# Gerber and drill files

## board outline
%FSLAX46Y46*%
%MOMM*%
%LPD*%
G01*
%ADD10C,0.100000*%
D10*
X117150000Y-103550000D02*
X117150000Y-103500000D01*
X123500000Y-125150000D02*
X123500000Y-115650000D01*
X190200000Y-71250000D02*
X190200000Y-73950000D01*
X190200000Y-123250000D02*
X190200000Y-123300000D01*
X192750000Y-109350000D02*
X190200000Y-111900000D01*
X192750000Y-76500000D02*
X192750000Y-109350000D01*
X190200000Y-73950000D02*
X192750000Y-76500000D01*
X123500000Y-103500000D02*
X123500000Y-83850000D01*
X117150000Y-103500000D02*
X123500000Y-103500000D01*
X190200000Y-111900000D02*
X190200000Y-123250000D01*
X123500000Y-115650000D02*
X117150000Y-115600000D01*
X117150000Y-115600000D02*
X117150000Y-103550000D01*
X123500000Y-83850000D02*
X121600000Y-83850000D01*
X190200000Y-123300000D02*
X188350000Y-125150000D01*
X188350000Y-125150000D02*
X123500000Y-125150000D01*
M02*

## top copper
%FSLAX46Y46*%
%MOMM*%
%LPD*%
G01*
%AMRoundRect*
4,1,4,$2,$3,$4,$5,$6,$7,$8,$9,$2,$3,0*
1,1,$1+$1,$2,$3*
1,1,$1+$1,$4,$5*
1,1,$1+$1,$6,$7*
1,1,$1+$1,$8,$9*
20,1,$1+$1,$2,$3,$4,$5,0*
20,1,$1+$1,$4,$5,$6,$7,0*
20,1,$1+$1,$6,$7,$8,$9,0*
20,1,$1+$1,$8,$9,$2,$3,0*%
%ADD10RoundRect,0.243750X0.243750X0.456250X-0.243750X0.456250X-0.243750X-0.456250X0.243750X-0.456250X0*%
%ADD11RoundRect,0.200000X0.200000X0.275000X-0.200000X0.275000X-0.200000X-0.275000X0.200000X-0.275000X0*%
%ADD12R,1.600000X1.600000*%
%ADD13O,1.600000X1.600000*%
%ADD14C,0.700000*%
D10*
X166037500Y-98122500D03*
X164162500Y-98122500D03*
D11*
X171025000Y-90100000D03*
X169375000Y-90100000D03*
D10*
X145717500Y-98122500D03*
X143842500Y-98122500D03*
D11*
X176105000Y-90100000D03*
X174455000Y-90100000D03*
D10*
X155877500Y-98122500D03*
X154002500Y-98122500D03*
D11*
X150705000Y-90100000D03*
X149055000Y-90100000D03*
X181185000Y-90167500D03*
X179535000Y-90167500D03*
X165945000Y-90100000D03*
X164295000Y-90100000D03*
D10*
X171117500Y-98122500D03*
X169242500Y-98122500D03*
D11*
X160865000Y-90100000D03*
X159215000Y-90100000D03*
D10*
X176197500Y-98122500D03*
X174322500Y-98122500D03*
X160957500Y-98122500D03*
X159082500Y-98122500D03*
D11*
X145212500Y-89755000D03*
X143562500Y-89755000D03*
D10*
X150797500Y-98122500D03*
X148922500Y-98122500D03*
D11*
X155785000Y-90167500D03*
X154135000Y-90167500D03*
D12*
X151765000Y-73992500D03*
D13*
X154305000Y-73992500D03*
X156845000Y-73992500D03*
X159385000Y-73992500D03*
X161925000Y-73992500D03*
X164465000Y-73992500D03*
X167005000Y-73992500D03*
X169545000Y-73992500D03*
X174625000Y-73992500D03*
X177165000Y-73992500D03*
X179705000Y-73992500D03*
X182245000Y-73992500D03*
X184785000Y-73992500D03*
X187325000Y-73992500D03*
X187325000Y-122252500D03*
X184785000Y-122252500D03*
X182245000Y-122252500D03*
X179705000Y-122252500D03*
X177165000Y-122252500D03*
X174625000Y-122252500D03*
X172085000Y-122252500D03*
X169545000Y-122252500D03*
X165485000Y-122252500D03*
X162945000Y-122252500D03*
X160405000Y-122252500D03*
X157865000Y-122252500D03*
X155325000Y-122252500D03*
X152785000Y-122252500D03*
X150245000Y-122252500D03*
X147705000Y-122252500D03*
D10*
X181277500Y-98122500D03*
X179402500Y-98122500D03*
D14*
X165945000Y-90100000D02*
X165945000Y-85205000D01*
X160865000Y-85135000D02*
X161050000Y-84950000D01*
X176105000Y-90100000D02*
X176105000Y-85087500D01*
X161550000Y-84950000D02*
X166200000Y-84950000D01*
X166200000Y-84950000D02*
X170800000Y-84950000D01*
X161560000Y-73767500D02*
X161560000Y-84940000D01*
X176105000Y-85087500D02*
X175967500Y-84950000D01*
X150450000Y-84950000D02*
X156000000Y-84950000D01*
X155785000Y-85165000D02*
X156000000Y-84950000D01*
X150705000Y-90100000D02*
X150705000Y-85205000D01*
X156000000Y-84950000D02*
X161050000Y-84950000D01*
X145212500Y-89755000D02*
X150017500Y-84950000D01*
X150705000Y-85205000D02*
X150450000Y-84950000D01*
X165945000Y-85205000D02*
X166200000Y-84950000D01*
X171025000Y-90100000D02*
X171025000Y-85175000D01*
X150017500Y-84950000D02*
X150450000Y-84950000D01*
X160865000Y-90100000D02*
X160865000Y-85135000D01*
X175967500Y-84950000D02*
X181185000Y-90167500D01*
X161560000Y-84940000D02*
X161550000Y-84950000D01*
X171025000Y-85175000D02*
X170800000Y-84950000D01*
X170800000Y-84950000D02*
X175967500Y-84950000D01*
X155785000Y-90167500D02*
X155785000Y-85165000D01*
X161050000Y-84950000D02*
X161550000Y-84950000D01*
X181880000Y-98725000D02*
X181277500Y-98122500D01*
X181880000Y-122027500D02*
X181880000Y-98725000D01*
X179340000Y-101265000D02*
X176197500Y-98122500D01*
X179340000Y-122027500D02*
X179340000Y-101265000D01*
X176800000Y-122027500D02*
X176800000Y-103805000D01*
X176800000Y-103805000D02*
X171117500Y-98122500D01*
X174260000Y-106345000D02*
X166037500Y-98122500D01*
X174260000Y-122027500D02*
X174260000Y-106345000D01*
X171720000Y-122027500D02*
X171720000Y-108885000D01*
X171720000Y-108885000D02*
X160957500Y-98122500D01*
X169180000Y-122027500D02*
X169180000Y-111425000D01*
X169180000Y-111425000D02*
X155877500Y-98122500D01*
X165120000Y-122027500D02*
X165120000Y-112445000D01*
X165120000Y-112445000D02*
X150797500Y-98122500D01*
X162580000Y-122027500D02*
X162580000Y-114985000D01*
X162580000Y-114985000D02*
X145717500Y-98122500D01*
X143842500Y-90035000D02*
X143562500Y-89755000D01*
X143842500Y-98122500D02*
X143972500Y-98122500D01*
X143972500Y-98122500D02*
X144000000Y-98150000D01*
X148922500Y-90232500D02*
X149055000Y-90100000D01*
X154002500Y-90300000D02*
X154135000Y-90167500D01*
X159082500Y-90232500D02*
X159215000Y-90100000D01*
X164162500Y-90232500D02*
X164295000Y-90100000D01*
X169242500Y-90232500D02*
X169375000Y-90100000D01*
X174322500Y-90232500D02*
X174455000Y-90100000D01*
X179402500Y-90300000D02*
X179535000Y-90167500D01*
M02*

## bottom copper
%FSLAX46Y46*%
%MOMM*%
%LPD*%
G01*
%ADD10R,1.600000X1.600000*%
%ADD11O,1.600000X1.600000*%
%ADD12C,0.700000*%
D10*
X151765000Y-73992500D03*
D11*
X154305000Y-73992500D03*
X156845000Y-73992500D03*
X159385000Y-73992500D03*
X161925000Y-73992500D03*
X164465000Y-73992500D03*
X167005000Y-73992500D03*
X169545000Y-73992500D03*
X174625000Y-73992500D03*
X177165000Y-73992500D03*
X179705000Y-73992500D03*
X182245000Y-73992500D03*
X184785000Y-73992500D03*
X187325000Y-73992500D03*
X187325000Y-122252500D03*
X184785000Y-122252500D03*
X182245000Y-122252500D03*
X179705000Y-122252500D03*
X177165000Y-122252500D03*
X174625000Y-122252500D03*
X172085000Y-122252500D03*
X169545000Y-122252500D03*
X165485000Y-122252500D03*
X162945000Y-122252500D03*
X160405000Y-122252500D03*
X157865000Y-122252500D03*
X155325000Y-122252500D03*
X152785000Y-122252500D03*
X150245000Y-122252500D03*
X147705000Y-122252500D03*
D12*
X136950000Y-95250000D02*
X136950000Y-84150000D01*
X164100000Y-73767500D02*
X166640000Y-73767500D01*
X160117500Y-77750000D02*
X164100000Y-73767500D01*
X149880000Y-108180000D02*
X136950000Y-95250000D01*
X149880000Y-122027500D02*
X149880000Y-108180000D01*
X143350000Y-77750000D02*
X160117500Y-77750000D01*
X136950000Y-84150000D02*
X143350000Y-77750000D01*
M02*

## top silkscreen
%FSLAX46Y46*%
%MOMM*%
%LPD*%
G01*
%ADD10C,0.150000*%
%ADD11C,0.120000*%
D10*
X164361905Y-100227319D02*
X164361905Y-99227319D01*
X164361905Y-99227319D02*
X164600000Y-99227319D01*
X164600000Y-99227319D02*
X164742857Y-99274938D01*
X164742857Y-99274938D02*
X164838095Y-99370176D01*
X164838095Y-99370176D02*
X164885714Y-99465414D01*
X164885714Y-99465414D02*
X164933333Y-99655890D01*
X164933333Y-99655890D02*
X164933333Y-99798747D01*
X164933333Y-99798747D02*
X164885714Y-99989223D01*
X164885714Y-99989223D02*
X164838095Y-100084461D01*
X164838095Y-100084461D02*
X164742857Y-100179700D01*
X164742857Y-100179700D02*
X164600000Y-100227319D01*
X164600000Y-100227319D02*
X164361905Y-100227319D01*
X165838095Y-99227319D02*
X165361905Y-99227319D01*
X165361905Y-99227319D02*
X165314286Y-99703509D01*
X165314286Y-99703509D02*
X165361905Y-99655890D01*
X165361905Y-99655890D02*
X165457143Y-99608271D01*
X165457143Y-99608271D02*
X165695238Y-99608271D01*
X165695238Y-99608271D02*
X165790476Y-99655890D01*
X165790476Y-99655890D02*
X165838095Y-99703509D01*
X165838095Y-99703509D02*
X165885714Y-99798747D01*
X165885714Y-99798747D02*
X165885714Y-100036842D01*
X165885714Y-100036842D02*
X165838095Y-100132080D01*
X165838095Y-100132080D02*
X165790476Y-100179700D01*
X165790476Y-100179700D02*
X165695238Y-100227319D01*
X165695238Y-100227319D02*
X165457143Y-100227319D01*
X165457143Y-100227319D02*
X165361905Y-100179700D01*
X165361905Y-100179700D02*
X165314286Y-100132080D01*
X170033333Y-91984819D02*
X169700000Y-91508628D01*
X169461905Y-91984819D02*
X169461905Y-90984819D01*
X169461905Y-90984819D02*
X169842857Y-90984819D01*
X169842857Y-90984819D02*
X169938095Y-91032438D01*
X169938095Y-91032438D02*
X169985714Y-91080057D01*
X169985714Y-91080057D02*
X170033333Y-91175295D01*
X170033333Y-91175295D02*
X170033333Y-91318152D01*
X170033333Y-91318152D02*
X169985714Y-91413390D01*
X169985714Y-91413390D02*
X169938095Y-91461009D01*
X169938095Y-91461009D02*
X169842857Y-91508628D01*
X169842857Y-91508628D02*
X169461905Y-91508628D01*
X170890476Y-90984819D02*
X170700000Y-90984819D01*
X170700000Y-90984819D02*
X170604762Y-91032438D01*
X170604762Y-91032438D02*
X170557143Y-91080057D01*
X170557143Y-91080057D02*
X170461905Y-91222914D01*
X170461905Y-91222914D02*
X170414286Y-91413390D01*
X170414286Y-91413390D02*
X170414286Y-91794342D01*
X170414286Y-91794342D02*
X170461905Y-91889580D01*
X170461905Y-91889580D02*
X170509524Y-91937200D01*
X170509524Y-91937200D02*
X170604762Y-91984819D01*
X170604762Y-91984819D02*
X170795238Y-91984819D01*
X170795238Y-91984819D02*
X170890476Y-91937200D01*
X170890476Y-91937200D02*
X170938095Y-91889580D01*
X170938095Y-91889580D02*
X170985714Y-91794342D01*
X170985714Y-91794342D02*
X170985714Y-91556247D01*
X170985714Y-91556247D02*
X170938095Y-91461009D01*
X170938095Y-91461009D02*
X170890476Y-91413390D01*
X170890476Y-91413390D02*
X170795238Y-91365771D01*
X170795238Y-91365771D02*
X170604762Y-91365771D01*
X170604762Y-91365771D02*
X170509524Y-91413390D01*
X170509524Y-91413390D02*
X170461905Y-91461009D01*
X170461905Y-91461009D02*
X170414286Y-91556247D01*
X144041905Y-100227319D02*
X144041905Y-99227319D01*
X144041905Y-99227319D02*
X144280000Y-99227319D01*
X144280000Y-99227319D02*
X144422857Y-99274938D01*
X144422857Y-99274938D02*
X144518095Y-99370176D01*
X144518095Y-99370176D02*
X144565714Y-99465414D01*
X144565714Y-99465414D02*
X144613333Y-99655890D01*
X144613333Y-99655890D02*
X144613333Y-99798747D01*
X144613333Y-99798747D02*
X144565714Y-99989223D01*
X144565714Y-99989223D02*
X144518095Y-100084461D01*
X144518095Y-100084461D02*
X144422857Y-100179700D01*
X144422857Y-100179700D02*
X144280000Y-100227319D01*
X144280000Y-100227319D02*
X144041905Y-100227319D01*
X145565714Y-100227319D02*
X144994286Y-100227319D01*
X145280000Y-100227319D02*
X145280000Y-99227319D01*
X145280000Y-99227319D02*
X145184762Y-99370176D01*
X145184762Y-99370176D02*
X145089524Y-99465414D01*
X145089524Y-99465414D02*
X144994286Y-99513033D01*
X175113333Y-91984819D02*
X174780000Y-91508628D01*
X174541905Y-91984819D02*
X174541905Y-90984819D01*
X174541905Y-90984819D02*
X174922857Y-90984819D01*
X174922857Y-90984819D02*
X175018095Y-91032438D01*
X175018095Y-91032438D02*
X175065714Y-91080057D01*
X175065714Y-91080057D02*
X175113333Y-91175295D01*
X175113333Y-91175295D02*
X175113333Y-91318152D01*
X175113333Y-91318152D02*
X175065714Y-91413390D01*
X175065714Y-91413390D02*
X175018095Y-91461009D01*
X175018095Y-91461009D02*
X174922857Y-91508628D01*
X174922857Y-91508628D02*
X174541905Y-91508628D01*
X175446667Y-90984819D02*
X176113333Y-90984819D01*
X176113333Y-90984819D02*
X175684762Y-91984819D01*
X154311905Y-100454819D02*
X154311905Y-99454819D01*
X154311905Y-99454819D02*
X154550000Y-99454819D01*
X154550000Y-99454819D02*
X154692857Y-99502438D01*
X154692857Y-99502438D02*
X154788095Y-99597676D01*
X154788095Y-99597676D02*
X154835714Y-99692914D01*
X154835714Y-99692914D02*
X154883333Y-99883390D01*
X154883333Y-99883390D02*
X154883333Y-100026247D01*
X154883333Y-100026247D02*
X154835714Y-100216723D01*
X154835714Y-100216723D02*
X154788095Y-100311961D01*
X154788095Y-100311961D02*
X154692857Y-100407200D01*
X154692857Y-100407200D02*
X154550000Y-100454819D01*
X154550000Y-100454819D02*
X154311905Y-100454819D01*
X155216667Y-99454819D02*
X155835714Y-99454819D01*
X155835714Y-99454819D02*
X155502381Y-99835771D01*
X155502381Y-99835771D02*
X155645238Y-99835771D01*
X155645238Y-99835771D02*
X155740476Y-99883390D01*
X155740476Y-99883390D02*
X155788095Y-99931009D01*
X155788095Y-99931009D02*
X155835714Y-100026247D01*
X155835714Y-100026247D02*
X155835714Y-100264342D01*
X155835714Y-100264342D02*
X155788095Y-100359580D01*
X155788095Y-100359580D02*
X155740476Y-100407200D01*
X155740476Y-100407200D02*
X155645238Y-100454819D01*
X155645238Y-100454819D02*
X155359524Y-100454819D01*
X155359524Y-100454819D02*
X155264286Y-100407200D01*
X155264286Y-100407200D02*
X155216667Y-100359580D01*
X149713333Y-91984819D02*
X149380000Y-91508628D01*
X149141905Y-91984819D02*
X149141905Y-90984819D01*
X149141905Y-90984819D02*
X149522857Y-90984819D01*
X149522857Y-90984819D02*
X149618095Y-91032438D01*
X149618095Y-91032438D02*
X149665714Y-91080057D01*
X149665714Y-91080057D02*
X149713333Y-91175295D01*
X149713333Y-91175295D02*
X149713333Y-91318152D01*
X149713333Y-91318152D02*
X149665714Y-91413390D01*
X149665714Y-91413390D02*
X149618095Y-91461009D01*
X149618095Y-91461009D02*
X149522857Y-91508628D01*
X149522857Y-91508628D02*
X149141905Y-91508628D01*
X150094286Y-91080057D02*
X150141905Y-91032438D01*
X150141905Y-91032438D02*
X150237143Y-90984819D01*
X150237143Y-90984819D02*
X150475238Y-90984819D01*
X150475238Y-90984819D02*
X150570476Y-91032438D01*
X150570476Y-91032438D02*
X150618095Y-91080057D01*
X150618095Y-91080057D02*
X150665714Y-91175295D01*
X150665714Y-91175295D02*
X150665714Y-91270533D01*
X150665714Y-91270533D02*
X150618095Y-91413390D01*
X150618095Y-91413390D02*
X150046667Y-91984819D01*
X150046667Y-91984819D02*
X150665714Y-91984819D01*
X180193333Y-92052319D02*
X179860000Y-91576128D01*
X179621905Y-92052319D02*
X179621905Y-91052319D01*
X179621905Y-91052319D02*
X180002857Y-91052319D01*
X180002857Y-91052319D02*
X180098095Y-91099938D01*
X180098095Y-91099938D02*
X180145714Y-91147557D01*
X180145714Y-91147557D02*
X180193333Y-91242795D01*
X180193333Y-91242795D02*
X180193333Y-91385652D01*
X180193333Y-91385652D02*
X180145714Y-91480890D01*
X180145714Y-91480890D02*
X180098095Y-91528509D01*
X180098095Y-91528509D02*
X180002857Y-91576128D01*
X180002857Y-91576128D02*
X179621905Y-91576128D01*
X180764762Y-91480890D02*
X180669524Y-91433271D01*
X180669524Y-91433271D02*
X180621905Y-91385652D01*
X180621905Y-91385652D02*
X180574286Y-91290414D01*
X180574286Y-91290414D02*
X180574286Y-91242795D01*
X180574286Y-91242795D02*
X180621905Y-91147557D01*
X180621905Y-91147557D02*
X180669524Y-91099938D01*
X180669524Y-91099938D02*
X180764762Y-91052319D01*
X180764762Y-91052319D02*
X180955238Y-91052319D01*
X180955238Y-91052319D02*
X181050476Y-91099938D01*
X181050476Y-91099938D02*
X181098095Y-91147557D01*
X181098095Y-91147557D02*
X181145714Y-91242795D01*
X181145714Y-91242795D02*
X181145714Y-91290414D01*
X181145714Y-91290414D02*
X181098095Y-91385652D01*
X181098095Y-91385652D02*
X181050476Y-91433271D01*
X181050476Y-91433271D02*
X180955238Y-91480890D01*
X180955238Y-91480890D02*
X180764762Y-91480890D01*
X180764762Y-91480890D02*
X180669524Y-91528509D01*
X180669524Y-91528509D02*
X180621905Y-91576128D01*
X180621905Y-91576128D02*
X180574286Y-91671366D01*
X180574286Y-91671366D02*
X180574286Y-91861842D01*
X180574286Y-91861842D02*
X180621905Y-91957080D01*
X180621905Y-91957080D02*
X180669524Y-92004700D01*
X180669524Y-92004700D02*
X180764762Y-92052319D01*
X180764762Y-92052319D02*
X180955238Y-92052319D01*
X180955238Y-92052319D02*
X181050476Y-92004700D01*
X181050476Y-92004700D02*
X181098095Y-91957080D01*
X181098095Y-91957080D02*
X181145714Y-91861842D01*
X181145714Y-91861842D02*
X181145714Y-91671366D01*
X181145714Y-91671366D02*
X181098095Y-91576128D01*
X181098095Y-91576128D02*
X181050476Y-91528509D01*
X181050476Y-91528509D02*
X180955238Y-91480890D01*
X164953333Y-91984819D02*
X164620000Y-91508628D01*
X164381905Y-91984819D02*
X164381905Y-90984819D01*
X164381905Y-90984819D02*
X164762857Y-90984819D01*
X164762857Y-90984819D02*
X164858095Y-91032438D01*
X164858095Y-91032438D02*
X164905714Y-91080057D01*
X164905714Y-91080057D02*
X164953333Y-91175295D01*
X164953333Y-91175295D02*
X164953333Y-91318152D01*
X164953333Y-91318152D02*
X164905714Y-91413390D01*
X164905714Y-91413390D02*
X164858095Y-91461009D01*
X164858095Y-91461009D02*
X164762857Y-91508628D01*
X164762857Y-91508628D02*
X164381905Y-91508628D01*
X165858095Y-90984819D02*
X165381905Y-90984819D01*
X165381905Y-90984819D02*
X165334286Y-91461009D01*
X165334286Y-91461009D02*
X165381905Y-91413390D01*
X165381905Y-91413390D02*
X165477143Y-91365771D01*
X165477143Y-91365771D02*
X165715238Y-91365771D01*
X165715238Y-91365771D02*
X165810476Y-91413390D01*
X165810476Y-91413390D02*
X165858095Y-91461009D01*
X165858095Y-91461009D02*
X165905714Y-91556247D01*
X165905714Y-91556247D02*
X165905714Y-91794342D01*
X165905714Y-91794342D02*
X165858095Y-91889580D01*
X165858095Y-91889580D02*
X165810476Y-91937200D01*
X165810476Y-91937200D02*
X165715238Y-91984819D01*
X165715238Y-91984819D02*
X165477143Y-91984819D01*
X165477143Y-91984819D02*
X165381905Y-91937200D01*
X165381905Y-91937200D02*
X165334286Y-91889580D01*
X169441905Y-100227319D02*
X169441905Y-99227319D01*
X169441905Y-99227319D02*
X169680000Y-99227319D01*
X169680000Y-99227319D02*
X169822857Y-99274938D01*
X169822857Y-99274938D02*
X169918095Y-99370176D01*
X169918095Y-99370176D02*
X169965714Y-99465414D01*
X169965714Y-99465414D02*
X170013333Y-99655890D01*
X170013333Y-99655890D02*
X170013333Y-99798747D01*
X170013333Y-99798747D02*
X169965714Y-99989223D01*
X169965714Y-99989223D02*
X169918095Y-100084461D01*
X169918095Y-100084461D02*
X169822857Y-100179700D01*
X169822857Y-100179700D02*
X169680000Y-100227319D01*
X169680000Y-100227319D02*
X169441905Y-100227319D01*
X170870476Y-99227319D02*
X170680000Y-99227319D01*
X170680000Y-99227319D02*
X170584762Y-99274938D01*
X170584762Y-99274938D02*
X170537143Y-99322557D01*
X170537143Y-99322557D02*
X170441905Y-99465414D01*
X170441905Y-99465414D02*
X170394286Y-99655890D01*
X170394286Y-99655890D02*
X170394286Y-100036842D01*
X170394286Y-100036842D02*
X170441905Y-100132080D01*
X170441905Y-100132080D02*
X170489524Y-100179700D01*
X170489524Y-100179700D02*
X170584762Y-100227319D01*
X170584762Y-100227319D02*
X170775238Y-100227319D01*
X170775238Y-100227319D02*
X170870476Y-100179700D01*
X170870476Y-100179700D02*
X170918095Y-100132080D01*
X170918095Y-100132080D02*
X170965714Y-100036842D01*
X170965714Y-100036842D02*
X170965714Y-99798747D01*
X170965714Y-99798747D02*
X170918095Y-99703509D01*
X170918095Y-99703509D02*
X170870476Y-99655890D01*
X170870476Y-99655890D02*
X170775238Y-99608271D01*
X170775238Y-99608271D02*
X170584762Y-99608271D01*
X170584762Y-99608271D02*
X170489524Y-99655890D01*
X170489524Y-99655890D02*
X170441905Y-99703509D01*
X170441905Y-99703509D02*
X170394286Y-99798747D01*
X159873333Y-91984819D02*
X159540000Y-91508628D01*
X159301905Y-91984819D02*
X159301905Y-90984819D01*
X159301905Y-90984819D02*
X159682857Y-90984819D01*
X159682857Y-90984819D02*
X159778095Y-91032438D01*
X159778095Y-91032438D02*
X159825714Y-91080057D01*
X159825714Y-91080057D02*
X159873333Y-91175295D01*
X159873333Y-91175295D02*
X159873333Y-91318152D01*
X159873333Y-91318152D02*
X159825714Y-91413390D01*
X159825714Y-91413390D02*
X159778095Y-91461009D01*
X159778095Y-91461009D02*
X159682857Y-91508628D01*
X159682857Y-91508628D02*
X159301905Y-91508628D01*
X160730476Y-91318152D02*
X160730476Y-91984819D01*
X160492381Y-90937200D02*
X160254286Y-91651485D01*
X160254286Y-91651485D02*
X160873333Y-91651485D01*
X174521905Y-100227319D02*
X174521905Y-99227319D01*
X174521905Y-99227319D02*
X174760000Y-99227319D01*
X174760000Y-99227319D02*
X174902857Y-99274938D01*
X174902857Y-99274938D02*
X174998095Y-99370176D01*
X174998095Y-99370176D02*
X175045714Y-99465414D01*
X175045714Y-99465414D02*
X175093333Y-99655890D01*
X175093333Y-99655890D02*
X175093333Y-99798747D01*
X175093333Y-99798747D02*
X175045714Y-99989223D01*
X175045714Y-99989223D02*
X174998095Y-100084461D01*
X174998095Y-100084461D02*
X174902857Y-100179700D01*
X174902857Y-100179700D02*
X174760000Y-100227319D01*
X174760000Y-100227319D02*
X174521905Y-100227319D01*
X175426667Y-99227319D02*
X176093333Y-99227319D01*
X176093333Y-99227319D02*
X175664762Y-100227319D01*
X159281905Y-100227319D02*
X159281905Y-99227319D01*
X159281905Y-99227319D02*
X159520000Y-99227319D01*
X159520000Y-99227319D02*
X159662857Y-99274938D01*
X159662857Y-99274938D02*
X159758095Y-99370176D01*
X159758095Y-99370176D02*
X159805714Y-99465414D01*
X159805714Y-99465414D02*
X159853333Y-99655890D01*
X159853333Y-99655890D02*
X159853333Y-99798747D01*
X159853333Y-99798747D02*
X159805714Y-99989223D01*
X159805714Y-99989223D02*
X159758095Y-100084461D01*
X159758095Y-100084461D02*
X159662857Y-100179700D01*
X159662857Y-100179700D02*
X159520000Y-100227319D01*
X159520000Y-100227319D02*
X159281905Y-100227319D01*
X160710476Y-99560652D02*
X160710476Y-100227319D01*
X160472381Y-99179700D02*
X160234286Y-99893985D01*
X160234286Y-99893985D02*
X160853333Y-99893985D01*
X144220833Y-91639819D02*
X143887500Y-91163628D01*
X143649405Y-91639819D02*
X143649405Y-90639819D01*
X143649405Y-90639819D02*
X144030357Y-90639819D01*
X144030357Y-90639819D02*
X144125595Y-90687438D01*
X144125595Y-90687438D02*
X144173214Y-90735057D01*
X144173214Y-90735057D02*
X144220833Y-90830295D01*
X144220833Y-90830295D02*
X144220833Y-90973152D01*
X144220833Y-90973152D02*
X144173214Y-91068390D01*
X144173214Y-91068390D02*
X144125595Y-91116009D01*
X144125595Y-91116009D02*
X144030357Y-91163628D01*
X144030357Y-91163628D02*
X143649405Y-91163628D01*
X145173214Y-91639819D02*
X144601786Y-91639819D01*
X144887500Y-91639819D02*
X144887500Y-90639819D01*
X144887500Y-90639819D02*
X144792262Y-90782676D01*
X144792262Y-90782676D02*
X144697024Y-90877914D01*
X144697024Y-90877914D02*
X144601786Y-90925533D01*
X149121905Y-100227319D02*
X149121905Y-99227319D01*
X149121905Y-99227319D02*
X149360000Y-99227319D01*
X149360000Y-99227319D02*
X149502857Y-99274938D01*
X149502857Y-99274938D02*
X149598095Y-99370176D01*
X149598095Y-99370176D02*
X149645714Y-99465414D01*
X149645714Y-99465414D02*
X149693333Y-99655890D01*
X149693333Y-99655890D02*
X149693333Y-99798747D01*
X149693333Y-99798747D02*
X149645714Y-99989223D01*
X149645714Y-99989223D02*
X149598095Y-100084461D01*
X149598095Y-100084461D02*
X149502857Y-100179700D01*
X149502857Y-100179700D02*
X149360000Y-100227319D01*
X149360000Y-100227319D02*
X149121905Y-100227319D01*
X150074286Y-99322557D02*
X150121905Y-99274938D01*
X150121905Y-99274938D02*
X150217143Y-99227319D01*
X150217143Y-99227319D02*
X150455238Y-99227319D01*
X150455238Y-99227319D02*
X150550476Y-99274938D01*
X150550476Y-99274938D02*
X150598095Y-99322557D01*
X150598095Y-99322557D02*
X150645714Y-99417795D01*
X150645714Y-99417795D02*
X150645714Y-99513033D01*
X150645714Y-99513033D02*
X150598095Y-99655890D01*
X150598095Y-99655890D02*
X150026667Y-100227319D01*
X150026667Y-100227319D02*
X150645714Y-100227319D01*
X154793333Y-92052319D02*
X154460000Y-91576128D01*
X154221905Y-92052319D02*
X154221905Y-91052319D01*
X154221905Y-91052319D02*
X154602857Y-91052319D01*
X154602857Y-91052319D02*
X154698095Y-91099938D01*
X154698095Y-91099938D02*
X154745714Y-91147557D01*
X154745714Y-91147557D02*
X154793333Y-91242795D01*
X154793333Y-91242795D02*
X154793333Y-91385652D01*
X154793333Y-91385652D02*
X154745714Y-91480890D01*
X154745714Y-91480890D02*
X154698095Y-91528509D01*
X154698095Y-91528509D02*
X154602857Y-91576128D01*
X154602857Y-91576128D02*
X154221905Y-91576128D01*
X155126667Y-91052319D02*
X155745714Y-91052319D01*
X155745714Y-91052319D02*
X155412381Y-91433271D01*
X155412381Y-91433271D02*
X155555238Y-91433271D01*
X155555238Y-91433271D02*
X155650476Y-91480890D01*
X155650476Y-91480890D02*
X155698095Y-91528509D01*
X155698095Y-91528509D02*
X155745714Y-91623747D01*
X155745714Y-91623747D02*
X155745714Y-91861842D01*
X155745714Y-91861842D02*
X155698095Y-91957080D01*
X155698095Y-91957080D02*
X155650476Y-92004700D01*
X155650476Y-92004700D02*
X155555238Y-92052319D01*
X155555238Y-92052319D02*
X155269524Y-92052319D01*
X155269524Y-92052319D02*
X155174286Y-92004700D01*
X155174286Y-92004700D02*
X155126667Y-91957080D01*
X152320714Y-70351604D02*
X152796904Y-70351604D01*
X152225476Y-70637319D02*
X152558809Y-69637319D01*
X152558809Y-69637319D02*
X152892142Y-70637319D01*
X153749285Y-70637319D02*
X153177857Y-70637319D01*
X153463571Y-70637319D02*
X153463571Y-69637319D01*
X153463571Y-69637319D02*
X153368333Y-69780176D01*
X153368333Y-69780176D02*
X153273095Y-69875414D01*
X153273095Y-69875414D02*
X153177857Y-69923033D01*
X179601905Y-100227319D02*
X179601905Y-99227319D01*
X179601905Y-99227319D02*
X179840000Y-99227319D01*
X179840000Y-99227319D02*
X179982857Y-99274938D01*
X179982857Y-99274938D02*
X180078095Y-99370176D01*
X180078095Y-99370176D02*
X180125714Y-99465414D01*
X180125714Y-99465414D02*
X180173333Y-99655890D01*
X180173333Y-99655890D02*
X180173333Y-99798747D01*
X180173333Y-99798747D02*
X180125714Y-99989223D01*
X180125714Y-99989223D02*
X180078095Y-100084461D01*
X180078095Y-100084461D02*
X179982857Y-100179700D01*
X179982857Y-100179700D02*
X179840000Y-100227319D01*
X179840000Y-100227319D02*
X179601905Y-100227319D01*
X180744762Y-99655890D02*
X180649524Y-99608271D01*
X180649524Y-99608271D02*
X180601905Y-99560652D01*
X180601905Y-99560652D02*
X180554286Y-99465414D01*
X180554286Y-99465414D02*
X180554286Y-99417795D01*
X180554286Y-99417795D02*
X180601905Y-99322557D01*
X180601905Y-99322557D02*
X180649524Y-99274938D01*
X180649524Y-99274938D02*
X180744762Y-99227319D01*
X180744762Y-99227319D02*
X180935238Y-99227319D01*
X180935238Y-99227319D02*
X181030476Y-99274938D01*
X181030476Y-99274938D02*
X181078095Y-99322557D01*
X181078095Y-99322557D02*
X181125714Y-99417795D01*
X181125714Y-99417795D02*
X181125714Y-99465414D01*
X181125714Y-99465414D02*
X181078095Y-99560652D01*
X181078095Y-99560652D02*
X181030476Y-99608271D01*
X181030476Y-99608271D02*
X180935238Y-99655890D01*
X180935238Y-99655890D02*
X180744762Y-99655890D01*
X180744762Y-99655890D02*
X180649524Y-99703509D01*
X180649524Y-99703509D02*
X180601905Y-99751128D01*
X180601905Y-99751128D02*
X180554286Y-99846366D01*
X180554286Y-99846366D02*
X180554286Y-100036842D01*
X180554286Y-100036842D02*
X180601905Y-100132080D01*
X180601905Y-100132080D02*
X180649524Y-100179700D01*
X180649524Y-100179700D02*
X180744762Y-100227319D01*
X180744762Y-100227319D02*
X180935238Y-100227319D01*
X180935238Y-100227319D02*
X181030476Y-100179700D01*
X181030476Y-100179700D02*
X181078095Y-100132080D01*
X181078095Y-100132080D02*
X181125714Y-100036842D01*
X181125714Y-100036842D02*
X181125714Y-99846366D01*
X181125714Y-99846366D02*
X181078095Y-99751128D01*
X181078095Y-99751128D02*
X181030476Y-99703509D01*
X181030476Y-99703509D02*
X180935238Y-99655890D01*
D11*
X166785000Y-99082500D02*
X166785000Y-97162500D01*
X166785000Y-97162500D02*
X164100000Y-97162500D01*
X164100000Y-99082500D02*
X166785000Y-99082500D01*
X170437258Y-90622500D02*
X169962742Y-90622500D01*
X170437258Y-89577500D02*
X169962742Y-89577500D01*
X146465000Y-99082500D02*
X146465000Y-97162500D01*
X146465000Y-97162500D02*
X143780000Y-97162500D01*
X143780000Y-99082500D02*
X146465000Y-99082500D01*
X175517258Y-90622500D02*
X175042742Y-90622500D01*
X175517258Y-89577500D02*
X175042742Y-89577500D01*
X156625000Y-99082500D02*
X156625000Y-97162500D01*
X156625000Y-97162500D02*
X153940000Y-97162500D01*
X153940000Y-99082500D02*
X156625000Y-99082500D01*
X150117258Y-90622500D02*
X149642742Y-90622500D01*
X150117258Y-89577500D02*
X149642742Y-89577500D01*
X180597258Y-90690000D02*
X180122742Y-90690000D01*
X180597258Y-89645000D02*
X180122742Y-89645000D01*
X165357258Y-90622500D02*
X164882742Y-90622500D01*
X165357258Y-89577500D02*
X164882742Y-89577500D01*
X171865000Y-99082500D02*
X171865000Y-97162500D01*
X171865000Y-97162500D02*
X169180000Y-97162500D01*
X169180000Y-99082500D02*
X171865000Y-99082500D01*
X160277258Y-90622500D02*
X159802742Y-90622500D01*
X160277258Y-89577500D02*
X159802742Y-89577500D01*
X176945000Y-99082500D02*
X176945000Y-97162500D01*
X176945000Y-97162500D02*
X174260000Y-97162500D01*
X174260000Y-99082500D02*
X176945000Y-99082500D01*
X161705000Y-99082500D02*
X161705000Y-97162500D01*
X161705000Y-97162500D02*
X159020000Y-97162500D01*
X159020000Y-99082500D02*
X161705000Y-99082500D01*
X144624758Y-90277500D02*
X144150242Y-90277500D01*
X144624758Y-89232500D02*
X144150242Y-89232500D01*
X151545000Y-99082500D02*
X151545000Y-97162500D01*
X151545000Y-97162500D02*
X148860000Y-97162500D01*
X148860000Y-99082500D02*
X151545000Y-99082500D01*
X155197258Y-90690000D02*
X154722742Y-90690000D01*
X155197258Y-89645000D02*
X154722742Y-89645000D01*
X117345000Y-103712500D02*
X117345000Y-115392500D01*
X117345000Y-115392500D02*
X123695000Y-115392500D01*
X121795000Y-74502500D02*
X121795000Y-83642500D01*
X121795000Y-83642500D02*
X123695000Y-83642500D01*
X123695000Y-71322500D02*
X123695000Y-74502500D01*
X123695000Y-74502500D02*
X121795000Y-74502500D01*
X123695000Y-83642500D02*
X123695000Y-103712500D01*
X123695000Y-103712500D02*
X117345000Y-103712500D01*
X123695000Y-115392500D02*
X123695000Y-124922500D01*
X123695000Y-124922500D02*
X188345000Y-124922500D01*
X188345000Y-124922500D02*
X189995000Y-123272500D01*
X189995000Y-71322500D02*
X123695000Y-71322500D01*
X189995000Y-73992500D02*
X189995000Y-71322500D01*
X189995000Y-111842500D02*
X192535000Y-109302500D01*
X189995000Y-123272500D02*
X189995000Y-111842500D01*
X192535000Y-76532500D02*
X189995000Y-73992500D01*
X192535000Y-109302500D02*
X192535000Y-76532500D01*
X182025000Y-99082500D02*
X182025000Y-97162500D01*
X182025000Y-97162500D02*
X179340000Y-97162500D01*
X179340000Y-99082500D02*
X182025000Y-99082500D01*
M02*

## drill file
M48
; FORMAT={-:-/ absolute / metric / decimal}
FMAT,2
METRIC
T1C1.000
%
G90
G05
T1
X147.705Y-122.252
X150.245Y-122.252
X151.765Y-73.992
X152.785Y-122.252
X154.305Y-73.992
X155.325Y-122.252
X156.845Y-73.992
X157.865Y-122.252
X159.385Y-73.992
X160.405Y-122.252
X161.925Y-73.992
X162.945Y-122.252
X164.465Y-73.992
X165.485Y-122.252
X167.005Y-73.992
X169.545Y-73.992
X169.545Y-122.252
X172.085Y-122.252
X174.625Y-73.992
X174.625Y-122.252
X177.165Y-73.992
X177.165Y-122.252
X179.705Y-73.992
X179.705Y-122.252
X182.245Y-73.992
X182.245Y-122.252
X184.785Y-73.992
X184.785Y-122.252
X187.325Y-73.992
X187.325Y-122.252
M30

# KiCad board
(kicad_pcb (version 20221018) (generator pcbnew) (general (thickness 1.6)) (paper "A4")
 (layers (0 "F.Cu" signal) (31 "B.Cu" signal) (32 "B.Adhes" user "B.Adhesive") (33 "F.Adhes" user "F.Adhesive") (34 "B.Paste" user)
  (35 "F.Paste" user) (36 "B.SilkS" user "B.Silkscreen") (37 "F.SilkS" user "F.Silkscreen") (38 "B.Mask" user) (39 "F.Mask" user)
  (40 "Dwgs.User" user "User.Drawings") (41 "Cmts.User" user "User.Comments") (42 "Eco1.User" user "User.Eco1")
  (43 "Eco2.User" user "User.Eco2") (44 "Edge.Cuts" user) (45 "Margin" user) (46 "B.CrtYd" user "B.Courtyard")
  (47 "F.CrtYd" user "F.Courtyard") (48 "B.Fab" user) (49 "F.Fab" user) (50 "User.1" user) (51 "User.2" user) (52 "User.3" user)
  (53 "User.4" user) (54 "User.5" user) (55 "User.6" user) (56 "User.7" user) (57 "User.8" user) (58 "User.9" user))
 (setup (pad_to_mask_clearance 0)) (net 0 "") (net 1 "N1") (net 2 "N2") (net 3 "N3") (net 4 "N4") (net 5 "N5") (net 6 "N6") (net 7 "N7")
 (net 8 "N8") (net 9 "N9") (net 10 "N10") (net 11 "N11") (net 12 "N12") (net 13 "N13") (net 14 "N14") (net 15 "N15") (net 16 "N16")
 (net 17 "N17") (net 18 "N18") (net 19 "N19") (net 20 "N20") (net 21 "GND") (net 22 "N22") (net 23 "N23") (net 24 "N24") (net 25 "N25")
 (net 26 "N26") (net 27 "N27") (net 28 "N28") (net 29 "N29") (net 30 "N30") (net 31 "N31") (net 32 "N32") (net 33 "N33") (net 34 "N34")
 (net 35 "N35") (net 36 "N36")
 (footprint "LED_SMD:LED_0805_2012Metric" (layer "F.Cu") (at 165.1 98.1225 180)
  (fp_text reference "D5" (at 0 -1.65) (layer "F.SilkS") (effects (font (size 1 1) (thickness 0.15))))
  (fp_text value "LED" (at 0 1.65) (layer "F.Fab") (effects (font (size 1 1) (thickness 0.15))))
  (fp_line (start -1.685 -0.96) (end -1.685 0.96) (stroke (width 0.12) (type solid)) (layer "F.SilkS"))
  (fp_line (start -1.685 0.96) (end 1 0.96) (stroke (width 0.12) (type solid)) (layer "F.SilkS"))
  (fp_line (start 1 -0.96) (end -1.685 -0.96) (stroke (width 0.12) (type solid)) (layer "F.SilkS"))
  (pad "1" smd roundrect (at -0.9375 0 180) (size 0.975 1.4) (layers "F.Cu" "F.Paste" "F.Mask") (roundrect_rratio 0.25) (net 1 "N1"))
  (pad "2" smd roundrect (at 0.9375 0 180) (size 0.975 1.4) (layers "F.Cu" "F.Paste" "F.Mask") (roundrect_rratio 0.25) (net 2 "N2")))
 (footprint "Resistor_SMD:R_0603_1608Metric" (layer "F.Cu") (at 170.2 90.1 180)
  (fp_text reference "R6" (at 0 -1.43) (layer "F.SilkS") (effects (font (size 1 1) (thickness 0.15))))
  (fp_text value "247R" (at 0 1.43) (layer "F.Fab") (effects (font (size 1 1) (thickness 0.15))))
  (fp_line (start -0.237258 -0.5225) (end 0.237258 -0.5225) (stroke (width 0.12) (type solid)) (layer "F.SilkS"))
  (fp_line (start -0.237258 0.5225) (end 0.237258 0.5225) (stroke (width 0.12) (type solid)) (layer "F.SilkS"))
  (pad "1" smd roundrect (at -0.825 0 180) (size 0.8 0.95) (layers "F.Cu" "F.Paste" "F.Mask") (roundrect_rratio 0.25) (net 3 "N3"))
  (pad "2" smd roundrect (at 0.825 0 180) (size 0.8 0.95) (layers "F.Cu" "F.Paste" "F.Mask") (roundrect_rratio 0.25) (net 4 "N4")))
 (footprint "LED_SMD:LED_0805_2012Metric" (layer "F.Cu") (at 144.78 98.1225 180)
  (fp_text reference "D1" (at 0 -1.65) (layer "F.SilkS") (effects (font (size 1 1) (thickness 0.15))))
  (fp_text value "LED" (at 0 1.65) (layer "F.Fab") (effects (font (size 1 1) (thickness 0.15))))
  (fp_line (start -1.685 -0.96) (end -1.685 0.96) (stroke (width 0.12) (type solid)) (layer "F.SilkS"))
  (fp_line (start -1.685 0.96) (end 1 0.96) (stroke (width 0.12) (type solid)) (layer "F.SilkS"))
  (fp_line (start 1 -0.96) (end -1.685 -0.96) (stroke (width 0.12) (type solid)) (layer "F.SilkS"))
  (pad "1" smd roundrect (at -0.9375 0 180) (size 0.975 1.4) (layers "F.Cu" "F.Paste" "F.Mask") (roundrect_rratio 0.25) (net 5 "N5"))
  (pad "2" smd roundrect (at 0.9375 0 180) (size 0.975 1.4) (layers "F.Cu" "F.Paste" "F.Mask") (roundrect_rratio 0.25) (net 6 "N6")))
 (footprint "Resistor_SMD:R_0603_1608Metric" (layer "F.Cu") (at 175.28 90.1 180)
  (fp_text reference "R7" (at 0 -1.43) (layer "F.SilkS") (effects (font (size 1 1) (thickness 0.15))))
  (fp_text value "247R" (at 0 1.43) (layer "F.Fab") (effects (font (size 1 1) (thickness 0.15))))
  (fp_line (start -0.237258 -0.5225) (end 0.237258 -0.5225) (stroke (width 0.12) (type solid)) (layer "F.SilkS"))
  (fp_line (start -0.237258 0.5225) (end 0.237258 0.5225) (stroke (width 0.12) (type solid)) (layer "F.SilkS"))
  (pad "1" smd roundrect (at -0.825 0 180) (size 0.8 0.95) (layers "F.Cu" "F.Paste" "F.Mask") (roundrect_rratio 0.25) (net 3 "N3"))
  (pad "2" smd roundrect (at 0.825 0 180) (size 0.8 0.95) (layers "F.Cu" "F.Paste" "F.Mask") (roundrect_rratio 0.25) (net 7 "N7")))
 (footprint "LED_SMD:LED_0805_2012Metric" (layer "F.Cu") (at 154.94 98.1225 180)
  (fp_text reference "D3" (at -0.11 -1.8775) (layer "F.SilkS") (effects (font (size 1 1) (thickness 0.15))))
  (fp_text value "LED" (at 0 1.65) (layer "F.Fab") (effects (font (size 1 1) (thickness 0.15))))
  (fp_line (start -1.685 -0.96) (end -1.685 0.96) (stroke (width 0.12) (type solid)) (layer "F.SilkS"))
  (fp_line (start -1.685 0.96) (end 1 0.96) (stroke (width 0.12) (type solid)) (layer "F.SilkS"))
  (fp_line (start 1 -0.96) (end -1.685 -0.96) (stroke (width 0.12) (type solid)) (layer "F.SilkS"))
  (pad "1" smd roundrect (at -0.9375 0 180) (size 0.975 1.4) (layers "F.Cu" "F.Paste" "F.Mask") (roundrect_rratio 0.25) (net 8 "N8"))
  (pad "2" smd roundrect (at 0.9375 0 180) (size 0.975 1.4) (layers "F.Cu" "F.Paste" "F.Mask") (roundrect_rratio 0.25) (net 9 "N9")))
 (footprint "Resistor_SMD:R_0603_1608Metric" (layer "F.Cu") (at 149.88 90.1 180)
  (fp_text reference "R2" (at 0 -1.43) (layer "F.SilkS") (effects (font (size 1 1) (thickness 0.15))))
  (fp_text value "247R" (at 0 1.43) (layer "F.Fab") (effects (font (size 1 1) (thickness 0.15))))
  (fp_line (start -0.237258 -0.5225) (end 0.237258 -0.5225) (stroke (width 0.12) (type solid)) (layer "F.SilkS"))
  (fp_line (start -0.237258 0.5225) (end 0.237258 0.5225) (stroke (width 0.12) (type solid)) (layer "F.SilkS"))
  (pad "1" smd roundrect (at -0.825 0 180) (size 0.8 0.95) (layers "F.Cu" "F.Paste" "F.Mask") (roundrect_rratio 0.25) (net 3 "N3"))
  (pad "2" smd roundrect (at 0.825 0 180) (size 0.8 0.95) (layers "F.Cu" "F.Paste" "F.Mask") (roundrect_rratio 0.25) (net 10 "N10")))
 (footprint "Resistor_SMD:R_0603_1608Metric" (layer "F.Cu") (at 180.36 90.1675 180)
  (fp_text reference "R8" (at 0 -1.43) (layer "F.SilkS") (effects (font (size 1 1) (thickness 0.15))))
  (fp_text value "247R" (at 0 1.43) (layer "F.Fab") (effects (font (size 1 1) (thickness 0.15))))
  (fp_line (start -0.237258 -0.5225) (end 0.237258 -0.5225) (stroke (width 0.12) (type solid)) (layer "F.SilkS"))
  (fp_line (start -0.237258 0.5225) (end 0.237258 0.5225) (stroke (width 0.12) (type solid)) (layer "F.SilkS"))
  (pad "1" smd roundrect (at -0.825 0 180) (size 0.8 0.95) (layers "F.Cu" "F.Paste" "F.Mask") (roundrect_rratio 0.25) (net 3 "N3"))
  (pad "2" smd roundrect (at 0.825 0 180) (size 0.8 0.95) (layers "F.Cu" "F.Paste" "F.Mask") (roundrect_rratio 0.25) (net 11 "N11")))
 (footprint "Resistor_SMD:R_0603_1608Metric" (layer "F.Cu") (at 165.12 90.1 180)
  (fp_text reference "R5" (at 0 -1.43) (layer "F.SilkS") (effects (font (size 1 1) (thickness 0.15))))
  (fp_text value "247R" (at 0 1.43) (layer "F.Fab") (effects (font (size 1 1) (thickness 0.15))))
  (fp_line (start -0.237258 -0.5225) (end 0.237258 -0.5225) (stroke (width 0.12) (type solid)) (layer "F.SilkS"))
  (fp_line (start -0.237258 0.5225) (end 0.237258 0.5225) (stroke (width 0.12) (type solid)) (layer "F.SilkS"))
  (pad "1" smd roundrect (at -0.825 0 180) (size 0.8 0.95) (layers "F.Cu" "F.Paste" "F.Mask") (roundrect_rratio 0.25) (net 3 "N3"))
  (pad "2" smd roundrect (at 0.825 0 180) (size 0.8 0.95) (layers "F.Cu" "F.Paste" "F.Mask") (roundrect_rratio 0.25) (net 2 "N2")))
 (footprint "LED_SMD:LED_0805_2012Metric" (layer "F.Cu") (at 170.18 98.1225 180)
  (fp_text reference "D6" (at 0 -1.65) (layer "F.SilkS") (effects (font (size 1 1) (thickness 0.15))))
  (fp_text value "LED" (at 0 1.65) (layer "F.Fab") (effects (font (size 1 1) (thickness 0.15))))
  (fp_line (start -1.685 -0.96) (end -1.685 0.96) (stroke (width 0.12) (type solid)) (layer "F.SilkS"))
  (fp_line (start -1.685 0.96) (end 1 0.96) (stroke (width 0.12) (type solid)) (layer "F.SilkS"))
  (fp_line (start 1 -0.96) (end -1.685 -0.96) (stroke (width 0.12) (type solid)) (layer "F.SilkS"))
  (pad "1" smd roundrect (at -0.9375 0 180) (size 0.975 1.4) (layers "F.Cu" "F.Paste" "F.Mask") (roundrect_rratio 0.25) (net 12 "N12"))
  (pad "2" smd roundrect (at 0.9375 0 180) (size 0.975 1.4) (layers "F.Cu" "F.Paste" "F.Mask") (roundrect_rratio 0.25) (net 4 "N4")))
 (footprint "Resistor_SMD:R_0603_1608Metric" (layer "F.Cu") (at 160.04 90.1 180)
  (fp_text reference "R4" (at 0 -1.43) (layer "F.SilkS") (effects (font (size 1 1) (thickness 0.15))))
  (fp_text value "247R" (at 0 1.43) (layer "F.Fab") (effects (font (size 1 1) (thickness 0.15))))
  (fp_line (start -0.237258 -0.5225) (end 0.237258 -0.5225) (stroke (width 0.12) (type solid)) (layer "F.SilkS"))
  (fp_line (start -0.237258 0.5225) (end 0.237258 0.5225) (stroke (width 0.12) (type solid)) (layer "F.SilkS"))
  (pad "1" smd roundrect (at -0.825 0 180) (size 0.8 0.95) (layers "F.Cu" "F.Paste" "F.Mask") (roundrect_rratio 0.25) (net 3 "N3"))
  (pad "2" smd roundrect (at 0.825 0 180) (size 0.8 0.95) (layers "F.Cu" "F.Paste" "F.Mask") (roundrect_rratio 0.25) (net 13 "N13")))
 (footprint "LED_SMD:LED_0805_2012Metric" (layer "F.Cu") (at 175.26 98.1225 180)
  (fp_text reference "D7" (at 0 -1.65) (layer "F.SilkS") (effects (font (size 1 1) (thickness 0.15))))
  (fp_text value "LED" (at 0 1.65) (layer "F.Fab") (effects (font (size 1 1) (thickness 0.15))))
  (fp_line (start -1.685 -0.96) (end -1.685 0.96) (stroke (width 0.12) (type solid)) (layer "F.SilkS"))
  (fp_line (start -1.685 0.96) (end 1 0.96) (stroke (width 0.12) (type solid)) (layer "F.SilkS"))
  (fp_line (start 1 -0.96) (end -1.685 -0.96) (stroke (width 0.12) (type solid)) (layer "F.SilkS"))
  (pad "1" smd roundrect (at -0.9375 0 180) (size 0.975 1.4) (layers "F.Cu" "F.Paste" "F.Mask") (roundrect_rratio 0.25) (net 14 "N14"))
  (pad "2" smd roundrect (at 0.9375 0 180) (size 0.975 1.4) (layers "F.Cu" "F.Paste" "F.Mask") (roundrect_rratio 0.25) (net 7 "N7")))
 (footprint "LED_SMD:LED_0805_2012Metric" (layer "F.Cu") (at 160.02 98.1225 180)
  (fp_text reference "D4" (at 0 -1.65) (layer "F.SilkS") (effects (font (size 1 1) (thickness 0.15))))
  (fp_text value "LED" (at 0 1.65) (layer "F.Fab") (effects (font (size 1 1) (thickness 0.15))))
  (fp_line (start -1.685 -0.96) (end -1.685 0.96) (stroke (width 0.12) (type solid)) (layer "F.SilkS"))
  (fp_line (start -1.685 0.96) (end 1 0.96) (stroke (width 0.12) (type solid)) (layer "F.SilkS"))
  (fp_line (start 1 -0.96) (end -1.685 -0.96) (stroke (width 0.12) (type solid)) (layer "F.SilkS"))
  (pad "1" smd roundrect (at -0.9375 0 180) (size 0.975 1.4) (layers "F.Cu" "F.Paste" "F.Mask") (roundrect_rratio 0.25) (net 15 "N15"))
  (pad "2" smd roundrect (at 0.9375 0 180) (size 0.975 1.4) (layers "F.Cu" "F.Paste" "F.Mask") (roundrect_rratio 0.25) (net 13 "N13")))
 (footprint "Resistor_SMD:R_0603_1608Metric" (layer "F.Cu") (at 144.3875 89.755 180)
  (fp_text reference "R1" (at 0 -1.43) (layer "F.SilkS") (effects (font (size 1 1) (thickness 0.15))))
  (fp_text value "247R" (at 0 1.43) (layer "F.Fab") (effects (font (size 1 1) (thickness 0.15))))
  (fp_line (start -0.237258 -0.5225) (end 0.237258 -0.5225) (stroke (width 0.12) (type solid)) (layer "F.SilkS"))
  (fp_line (start -0.237258 0.5225) (end 0.237258 0.5225) (stroke (width 0.12) (type solid)) (layer "F.SilkS"))
  (pad "1" smd roundrect (at -0.825 0 180) (size 0.8 0.95) (layers "F.Cu" "F.Paste" "F.Mask") (roundrect_rratio 0.25) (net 3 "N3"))
  (pad "2" smd roundrect (at 0.825 0 180) (size 0.8 0.95) (layers "F.Cu" "F.Paste" "F.Mask") (roundrect_rratio 0.25) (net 6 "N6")))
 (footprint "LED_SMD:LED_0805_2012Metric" (layer "F.Cu") (at 149.86 98.1225 180)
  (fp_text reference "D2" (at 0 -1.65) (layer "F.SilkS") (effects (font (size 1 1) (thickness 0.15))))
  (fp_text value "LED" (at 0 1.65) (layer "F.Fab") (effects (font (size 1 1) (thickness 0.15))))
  (fp_line (start -1.685 -0.96) (end -1.685 0.96) (stroke (width 0.12) (type solid)) (layer "F.SilkS"))
  (fp_line (start -1.685 0.96) (end 1 0.96) (stroke (width 0.12) (type solid)) (layer "F.SilkS"))
  (fp_line (start 1 -0.96) (end -1.685 -0.96) (stroke (width 0.12) (type solid)) (layer "F.SilkS"))
  (pad "1" smd roundrect (at -0.9375 0 180) (size 0.975 1.4) (layers "F.Cu" "F.Paste" "F.Mask") (roundrect_rratio 0.25) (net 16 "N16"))
  (pad "2" smd roundrect (at 0.9375 0 180) (size 0.975 1.4) (layers "F.Cu" "F.Paste" "F.Mask") (roundrect_rratio 0.25) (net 10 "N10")))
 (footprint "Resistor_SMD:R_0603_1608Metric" (layer "F.Cu") (at 154.96 90.1675 180)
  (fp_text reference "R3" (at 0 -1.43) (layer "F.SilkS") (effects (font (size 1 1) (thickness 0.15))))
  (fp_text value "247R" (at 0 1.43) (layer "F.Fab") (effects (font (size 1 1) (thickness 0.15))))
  (fp_line (start -0.237258 -0.5225) (end 0.237258 -0.5225) (stroke (width 0.12) (type solid)) (layer "F.SilkS"))
  (fp_line (start -0.237258 0.5225) (end 0.237258 0.5225) (stroke (width 0.12) (type solid)) (layer "F.SilkS"))
  (pad "1" smd roundrect (at -0.825 0 180) (size 0.8 0.95) (layers "F.Cu" "F.Paste" "F.Mask") (roundrect_rratio 0.25) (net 3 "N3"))
  (pad "2" smd roundrect (at 0.825 0 180) (size 0.8 0.95) (layers "F.Cu" "F.Paste" "F.Mask") (roundrect_rratio 0.25) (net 9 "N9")))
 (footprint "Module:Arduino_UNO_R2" (layer "F.Cu") (at 151.765 73.9925)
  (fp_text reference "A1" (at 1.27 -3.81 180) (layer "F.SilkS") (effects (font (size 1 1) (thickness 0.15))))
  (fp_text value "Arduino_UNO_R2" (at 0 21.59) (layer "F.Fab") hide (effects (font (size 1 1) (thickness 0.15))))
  (fp_line (start -34.42 29.72) (end -34.42 41.4) (stroke (width 0.12) (type solid)) (layer "F.SilkS"))
  (fp_line (start -34.42 41.4) (end -28.07 41.4) (stroke (width 0.12) (type solid)) (layer "F.SilkS"))
  (fp_line (start -29.97 0.51) (end -29.97 9.65) (stroke (width 0.12) (type solid)) (layer "F.SilkS"))
  (fp_line (start -29.97 9.65) (end -28.07 9.65) (stroke (width 0.12) (type solid)) (layer "F.SilkS"))
  (fp_line (start -28.07 -2.67) (end -28.07 0.51) (stroke (width 0.12) (type solid)) (layer "F.SilkS"))
  (fp_line (start -28.07 0.51) (end -29.97 0.51) (stroke (width 0.12) (type solid)) (layer "F.SilkS"))
  (fp_line (start -28.07 9.65) (end -28.07 29.72) (stroke (width 0.12) (type solid)) (layer "F.SilkS"))
  (fp_line (start -28.07 29.72) (end -34.42 29.72) (stroke (width 0.12) (type solid)) (layer "F.SilkS"))
  (fp_line (start -28.07 41.4) (end -28.07 50.93) (stroke (width 0.12) (type solid)) (layer "F.SilkS"))
  (fp_line (start -28.07 50.93) (end 36.58 50.93) (stroke (width 0.12) (type solid)) (layer "F.SilkS"))
  (fp_line (start 36.58 50.93) (end 38.23 49.28) (stroke (width 0.12) (type solid)) (layer "F.SilkS"))
  (fp_line (start 38.23 -2.67) (end -28.07 -2.67) (stroke (width 0.12) (type solid)) (layer "F.SilkS"))
  (fp_line (start 38.23 0) (end 38.23 -2.67) (stroke (width 0.12) (type solid)) (layer "F.SilkS"))
  (fp_line (start 38.23 37.85) (end 40.77 35.31) (stroke (width 0.12) (type solid)) (layer "F.SilkS"))
  (fp_line (start 38.23 49.28) (end 38.23 37.85) (stroke (width 0.12) (type solid)) (layer "F.SilkS"))
  (fp_line (start 40.77 2.54) (end 38.23 0) (stroke (width 0.12) (type solid)) (layer "F.SilkS"))
  (fp_line (start 40.77 35.31) (end 40.77 2.54) (stroke (width 0.12) (type solid)) (layer "F.SilkS"))
  (pad "1" thru_hole rect (at 0 0 90) (size 1.6 1.6) (drill 1) (layers "*.Cu" "*.Mask") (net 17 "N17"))
  (pad "2" thru_hole oval (at 2.54 0 90) (size 1.6 1.6) (drill 1) (layers "*.Cu" "*.Mask") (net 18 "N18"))
  (pad "3" thru_hole oval (at 5.08 0 90) (size 1.6 1.6) (drill 1) (layers "*.Cu" "*.Mask") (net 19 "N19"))
  (pad "4" thru_hole oval (at 7.62 0 90) (size 1.6 1.6) (drill 1) (layers "*.Cu" "*.Mask") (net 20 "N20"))
  (pad "5" thru_hole oval (at 10.16 0 90) (size 1.6 1.6) (drill 1) (layers "*.Cu" "*.Mask") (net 3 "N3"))
  (pad "6" thru_hole oval (at 12.7 0 90) (size 1.6 1.6) (drill 1) (layers "*.Cu" "*.Mask") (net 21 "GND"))
  (pad "7" thru_hole oval (at 15.24 0 90) (size 1.6 1.6) (drill 1) (layers "*.Cu" "*.Mask") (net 21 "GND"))
  (pad "8" thru_hole oval (at 17.78 0 90) (size 1.6 1.6) (drill 1) (layers "*.Cu" "*.Mask") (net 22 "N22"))
  (pad "9" thru_hole oval (at 22.86 0 90) (size 1.6 1.6) (drill 1) (layers "*.Cu" "*.Mask") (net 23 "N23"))
  (pad "10" thru_hole oval (at 25.4 0 90) (size 1.6 1.6) (drill 1) (layers "*.Cu" "*.Mask") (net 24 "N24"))
  (pad "11" thru_hole oval (at 27.94 0 90) (size 1.6 1.6) (drill 1) (layers "*.Cu" "*.Mask") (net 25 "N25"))
  (pad "12" thru_hole oval (at 30.48 0 90) (size 1.6 1.6) (drill 1) (layers "*.Cu" "*.Mask") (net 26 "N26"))
  (pad "13" thru_hole oval (at 33.02 0 90) (size 1.6 1.6) (drill 1) (layers "*.Cu" "*.Mask") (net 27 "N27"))
  (pad "14" thru_hole oval (at 35.56 0 90) (size 1.6 1.6) (drill 1) (layers "*.Cu" "*.Mask") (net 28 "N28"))
  (pad "15" thru_hole oval (at 35.56 48.26 90) (size 1.6 1.6) (drill 1) (layers "*.Cu" "*.Mask") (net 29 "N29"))
  (pad "16" thru_hole oval (at 33.02 48.26 90) (size 1.6 1.6) (drill 1) (layers "*.Cu" "*.Mask") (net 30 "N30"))
  (pad "17" thru_hole oval (at 30.48 48.26 90) (size 1.6 1.6) (drill 1) (layers "*.Cu" "*.Mask") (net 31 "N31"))
  (pad "18" thru_hole oval (at 27.94 48.26 90) (size 1.6 1.6) (drill 1) (layers "*.Cu" "*.Mask") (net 14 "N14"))
  (pad "19" thru_hole oval (at 25.4 48.26 90) (size 1.6 1.6) (drill 1) (layers "*.Cu" "*.Mask") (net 12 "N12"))
  (pad "20" thru_hole oval (at 22.86 48.26 90) (size 1.6 1.6) (drill 1) (layers "*.Cu" "*.Mask") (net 1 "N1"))
  (pad "21" thru_hole oval (at 20.32 48.26 90) (size 1.6 1.6) (drill 1) (layers "*.Cu" "*.Mask") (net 15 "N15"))
  (pad "22" thru_hole oval (at 17.78 48.26 90) (size 1.6 1.6) (drill 1) (layers "*.Cu" "*.Mask") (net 8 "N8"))
  (pad "23" thru_hole oval (at 13.72 48.26 90) (size 1.6 1.6) (drill 1) (layers "*.Cu" "*.Mask") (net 16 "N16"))
  (pad "24" thru_hole oval (at 11.18 48.26 90) (size 1.6 1.6) (drill 1) (layers "*.Cu" "*.Mask") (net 5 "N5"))
  (pad "25" thru_hole oval (at 8.64 48.26 90) (size 1.6 1.6) (drill 1) (layers "*.Cu" "*.Mask") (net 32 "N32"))
  (pad "26" thru_hole oval (at 6.1 48.26 90) (size 1.6 1.6) (drill 1) (layers "*.Cu" "*.Mask") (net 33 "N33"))
  (pad "27" thru_hole oval (at 3.56 48.26 90) (size 1.6 1.6) (drill 1) (layers "*.Cu" "*.Mask") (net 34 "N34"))
  (pad "28" thru_hole oval (at 1.02 48.26 90) (size 1.6 1.6) (drill 1) (layers "*.Cu" "*.Mask") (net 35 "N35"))
  (pad "29" thru_hole oval (at -1.52 48.26 90) (size 1.6 1.6) (drill 1) (layers "*.Cu" "*.Mask") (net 21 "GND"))
  (pad "30" thru_hole oval (at -4.06 48.26 90) (size 1.6 1.6) (drill 1) (layers "*.Cu" "*.Mask") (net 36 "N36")))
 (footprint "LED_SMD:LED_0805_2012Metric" (layer "F.Cu") (at 180.34 98.1225 180)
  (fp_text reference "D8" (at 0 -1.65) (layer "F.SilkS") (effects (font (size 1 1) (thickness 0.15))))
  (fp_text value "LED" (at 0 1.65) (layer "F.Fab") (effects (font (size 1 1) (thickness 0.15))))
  (fp_line (start -1.685 -0.96) (end -1.685 0.96) (stroke (width 0.12) (type solid)) (layer "F.SilkS"))
  (fp_line (start -1.685 0.96) (end 1 0.96) (stroke (width 0.12) (type solid)) (layer "F.SilkS"))
  (fp_line (start 1 -0.96) (end -1.685 -0.96) (stroke (width 0.12) (type solid)) (layer "F.SilkS"))
  (pad "1" smd roundrect (at -0.9375 0 180) (size 0.975 1.4) (layers "F.Cu" "F.Paste" "F.Mask") (roundrect_rratio 0.25) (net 31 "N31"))
  (pad "2" smd roundrect (at 0.9375 0 180) (size 0.975 1.4) (layers "F.Cu" "F.Paste" "F.Mask") (roundrect_rratio 0.25) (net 11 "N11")))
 (gr_line (start 117.15 103.55) (end 117.15 103.5) (stroke (width 0.1) (type default)) (layer "Edge.Cuts"))
 (gr_line (start 123.5 125.15) (end 123.5 115.65) (stroke (width 0.1) (type default)) (layer "Edge.Cuts"))
 (gr_line (start 190.2 71.25) (end 190.2 73.95) (stroke (width 0.1) (type default)) (layer "Edge.Cuts"))
 (gr_line (start 190.2 123.25) (end 190.2 123.3) (stroke (width 0.1) (type default)) (layer "Edge.Cuts"))
 (gr_line (start 192.75 109.35) (end 190.2 111.9) (stroke (width 0.1) (type default)) (layer "Edge.Cuts"))
 (gr_line (start 192.75 76.5) (end 192.75 109.35) (stroke (width 0.1) (type default)) (layer "Edge.Cuts"))
 (gr_line (start 190.2 73.95) (end 192.75 76.5) (stroke (width 0.1) (type default)) (layer "Edge.Cuts"))
 (gr_line (start 123.5 103.5) (end 123.5 83.85) (stroke (width 0.1) (type default)) (layer "Edge.Cuts"))
 (gr_line (start 117.15 103.5) (end 123.5 103.5) (stroke (width 0.1) (type default)) (layer "Edge.Cuts"))
 (gr_line (start 190.2 111.9) (end 190.2 123.25) (stroke (width 0.1) (type default)) (layer "Edge.Cuts"))
 (gr_line (start 123.5 115.65) (end 117.15 115.6) (stroke (width 0.1) (type default)) (layer "Edge.Cuts"))
 (gr_line (start 117.15 115.6) (end 117.15 103.55) (stroke (width 0.1) (type default)) (layer "Edge.Cuts"))
 (gr_line (start 123.5 83.85) (end 121.6 83.85) (stroke (width 0.1) (type default)) (layer "Edge.Cuts"))
 (gr_line (start 190.2 123.3) (end 188.35 125.15) (stroke (width 0.1) (type default)) (layer "Edge.Cuts"))
 (gr_line (start 188.35 125.15) (end 123.5 125.15) (stroke (width 0.1) (type default)) (layer "Edge.Cuts"))
 (segment (start 165.945 90.1) (end 165.945 85.205) (width 0.7) (layer "F.Cu") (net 3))
 (segment (start 160.865 85.135) (end 161.05 84.95) (width 0.7) (layer "F.Cu") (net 3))
 (segment (start 176.105 90.1) (end 176.105 85.0875) (width 0.7) (layer "F.Cu") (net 3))
 (segment (start 161.55 84.95) (end 166.2 84.95) (width 0.7) (layer "F.Cu") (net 3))
 (segment (start 166.2 84.95) (end 170.8 84.95) (width 0.7) (layer "F.Cu") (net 3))
 (segment (start 161.56 73.7675) (end 161.56 84.94) (width 0.7) (layer "F.Cu") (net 3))
 (segment (start 176.105 85.0875) (end 175.9675 84.95) (width 0.7) (layer "F.Cu") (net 3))
 (segment (start 150.45 84.95) (end 156 84.95) (width 0.7) (layer "F.Cu") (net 3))
 (segment (start 155.785 85.165) (end 156 84.95) (width 0.7) (layer "F.Cu") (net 3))
 (segment (start 150.705 90.1) (end 150.705 85.205) (width 0.7) (layer "F.Cu") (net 3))
 (segment (start 156 84.95) (end 161.05 84.95) (width 0.7) (layer "F.Cu") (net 3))
 (segment (start 145.2125 89.755) (end 150.0175 84.95) (width 0.7) (layer "F.Cu") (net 3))
 (segment (start 150.705 85.205) (end 150.45 84.95) (width 0.7) (layer "F.Cu") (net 3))
 (segment (start 165.945 85.205) (end 166.2 84.95) (width 0.7) (layer "F.Cu") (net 3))
 (segment (start 171.025 90.1) (end 171.025 85.175) (width 0.7) (layer "F.Cu") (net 3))
 (segment (start 150.0175 84.95) (end 150.45 84.95) (width 0.7) (layer "F.Cu") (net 3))
 (segment (start 160.865 90.1) (end 160.865 85.135) (width 0.7) (layer "F.Cu") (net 3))
 (segment (start 175.9675 84.95) (end 181.185 90.1675) (width 0.7) (layer "F.Cu") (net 3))
 (segment (start 161.56 84.94) (end 161.55 84.95) (width 0.7) (layer "F.Cu") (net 3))
 (segment (start 171.025 85.175) (end 170.8 84.95) (width 0.7) (layer "F.Cu") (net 3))
 (segment (start 170.8 84.95) (end 175.9675 84.95) (width 0.7) (layer "F.Cu") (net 3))
 (segment (start 155.785 90.1675) (end 155.785 85.165) (width 0.7) (layer "F.Cu") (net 3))
 (segment (start 161.05 84.95) (end 161.55 84.95) (width 0.7) (layer "F.Cu") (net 3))
 (segment (start 136.95 95.25) (end 136.95 84.15) (width 0.7) (layer "B.Cu") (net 21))
 (segment (start 164.1 73.7675) (end 166.64 73.7675) (width 0.7) (layer "B.Cu") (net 21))
 (segment (start 160.1175 77.75) (end 164.1 73.7675) (width 0.7) (layer "B.Cu") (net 21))
 (segment (start 149.88 108.18) (end 136.95 95.25) (width 0.7) (layer "B.Cu") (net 21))
 (segment (start 149.88 122.0275) (end 149.88 108.18) (width 0.7) (layer "B.Cu") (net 21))
 (segment (start 143.35 77.75) (end 160.1175 77.75) (width 0.7) (layer "B.Cu") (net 21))
 (segment (start 136.95 84.15) (end 143.35 77.75) (width 0.7) (layer "B.Cu") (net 21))
 (segment (start 181.88 98.725) (end 181.2775 98.1225) (width 0.7) (layer "F.Cu") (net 31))
 (segment (start 181.88 122.0275) (end 181.88 98.725) (width 0.7) (layer "F.Cu") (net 31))
 (segment (start 179.34 101.265) (end 176.1975 98.1225) (width 0.7) (layer "F.Cu") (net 14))
 (segment (start 179.34 122.0275) (end 179.34 101.265) (width 0.7) (layer "F.Cu") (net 14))
 (segment (start 176.8 122.0275) (end 176.8 103.805) (width 0.7) (layer "F.Cu") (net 12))
 (segment (start 176.8 103.805) (end 171.1175 98.1225) (width 0.7) (layer "F.Cu") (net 12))
 (segment (start 174.26 106.345) (end 166.0375 98.1225) (width 0.7) (layer "F.Cu") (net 1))
 (segment (start 174.26 122.0275) (end 174.26 106.345) (width 0.7) (layer "F.Cu") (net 1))
 (segment (start 171.72 122.0275) (end 171.72 108.885) (width 0.7) (layer "F.Cu") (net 15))
 (segment (start 171.72 108.885) (end 160.9575 98.1225) (width 0.7) (layer "F.Cu") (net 15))
 (segment (start 169.18 122.0275) (end 169.18 111.425) (width 0.7) (layer "F.Cu") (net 8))
 (segment (start 169.18 111.425) (end 155.8775 98.1225) (width 0.7) (layer "F.Cu") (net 8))
 (segment (start 165.12 122.0275) (end 165.12 112.445) (width 0.7) (layer "F.Cu") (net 16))
 (segment (start 165.12 112.445) (end 150.7975 98.1225) (width 0.7) (layer "F.Cu") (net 16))
 (segment (start 162.58 122.0275) (end 162.58 114.985) (width 0.7) (layer "F.Cu") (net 5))
 (segment (start 162.58 114.985) (end 145.7175 98.1225) (width 0.7) (layer "F.Cu") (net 5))
 (segment (start 143.8425 90.035) (end 143.5625 89.755) (width 0.7) (layer "F.Cu") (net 6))
 (segment (start 143.8425 98.1225) (end 143.9725 98.1225) (width 0.7) (layer "F.Cu") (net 6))
 (segment (start 143.9725 98.1225) (end 144 98.15) (width 0.7) (layer "F.Cu") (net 6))
 (segment (start 148.9225 90.2325) (end 149.055 90.1) (width 0.7) (layer "F.Cu") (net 10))
 (segment (start 154.0025 90.3) (end 154.135 90.1675) (width 0.7) (layer "F.Cu") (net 9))
 (segment (start 159.0825 90.2325) (end 159.215 90.1) (width 0.7) (layer "F.Cu") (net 13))
 (segment (start 164.1625 90.2325) (end 164.295 90.1) (width 0.7) (layer "F.Cu") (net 2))
 (segment (start 169.2425 90.2325) (end 169.375 90.1) (width 0.7) (layer "F.Cu") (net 4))
 (segment (start 174.3225 90.2325) (end 174.455 90.1) (width 0.7) (layer "F.Cu") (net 7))
 (segment (start 179.4025 90.3) (end 179.535 90.1675) (width 0.7) (layer "F.Cu") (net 11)))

